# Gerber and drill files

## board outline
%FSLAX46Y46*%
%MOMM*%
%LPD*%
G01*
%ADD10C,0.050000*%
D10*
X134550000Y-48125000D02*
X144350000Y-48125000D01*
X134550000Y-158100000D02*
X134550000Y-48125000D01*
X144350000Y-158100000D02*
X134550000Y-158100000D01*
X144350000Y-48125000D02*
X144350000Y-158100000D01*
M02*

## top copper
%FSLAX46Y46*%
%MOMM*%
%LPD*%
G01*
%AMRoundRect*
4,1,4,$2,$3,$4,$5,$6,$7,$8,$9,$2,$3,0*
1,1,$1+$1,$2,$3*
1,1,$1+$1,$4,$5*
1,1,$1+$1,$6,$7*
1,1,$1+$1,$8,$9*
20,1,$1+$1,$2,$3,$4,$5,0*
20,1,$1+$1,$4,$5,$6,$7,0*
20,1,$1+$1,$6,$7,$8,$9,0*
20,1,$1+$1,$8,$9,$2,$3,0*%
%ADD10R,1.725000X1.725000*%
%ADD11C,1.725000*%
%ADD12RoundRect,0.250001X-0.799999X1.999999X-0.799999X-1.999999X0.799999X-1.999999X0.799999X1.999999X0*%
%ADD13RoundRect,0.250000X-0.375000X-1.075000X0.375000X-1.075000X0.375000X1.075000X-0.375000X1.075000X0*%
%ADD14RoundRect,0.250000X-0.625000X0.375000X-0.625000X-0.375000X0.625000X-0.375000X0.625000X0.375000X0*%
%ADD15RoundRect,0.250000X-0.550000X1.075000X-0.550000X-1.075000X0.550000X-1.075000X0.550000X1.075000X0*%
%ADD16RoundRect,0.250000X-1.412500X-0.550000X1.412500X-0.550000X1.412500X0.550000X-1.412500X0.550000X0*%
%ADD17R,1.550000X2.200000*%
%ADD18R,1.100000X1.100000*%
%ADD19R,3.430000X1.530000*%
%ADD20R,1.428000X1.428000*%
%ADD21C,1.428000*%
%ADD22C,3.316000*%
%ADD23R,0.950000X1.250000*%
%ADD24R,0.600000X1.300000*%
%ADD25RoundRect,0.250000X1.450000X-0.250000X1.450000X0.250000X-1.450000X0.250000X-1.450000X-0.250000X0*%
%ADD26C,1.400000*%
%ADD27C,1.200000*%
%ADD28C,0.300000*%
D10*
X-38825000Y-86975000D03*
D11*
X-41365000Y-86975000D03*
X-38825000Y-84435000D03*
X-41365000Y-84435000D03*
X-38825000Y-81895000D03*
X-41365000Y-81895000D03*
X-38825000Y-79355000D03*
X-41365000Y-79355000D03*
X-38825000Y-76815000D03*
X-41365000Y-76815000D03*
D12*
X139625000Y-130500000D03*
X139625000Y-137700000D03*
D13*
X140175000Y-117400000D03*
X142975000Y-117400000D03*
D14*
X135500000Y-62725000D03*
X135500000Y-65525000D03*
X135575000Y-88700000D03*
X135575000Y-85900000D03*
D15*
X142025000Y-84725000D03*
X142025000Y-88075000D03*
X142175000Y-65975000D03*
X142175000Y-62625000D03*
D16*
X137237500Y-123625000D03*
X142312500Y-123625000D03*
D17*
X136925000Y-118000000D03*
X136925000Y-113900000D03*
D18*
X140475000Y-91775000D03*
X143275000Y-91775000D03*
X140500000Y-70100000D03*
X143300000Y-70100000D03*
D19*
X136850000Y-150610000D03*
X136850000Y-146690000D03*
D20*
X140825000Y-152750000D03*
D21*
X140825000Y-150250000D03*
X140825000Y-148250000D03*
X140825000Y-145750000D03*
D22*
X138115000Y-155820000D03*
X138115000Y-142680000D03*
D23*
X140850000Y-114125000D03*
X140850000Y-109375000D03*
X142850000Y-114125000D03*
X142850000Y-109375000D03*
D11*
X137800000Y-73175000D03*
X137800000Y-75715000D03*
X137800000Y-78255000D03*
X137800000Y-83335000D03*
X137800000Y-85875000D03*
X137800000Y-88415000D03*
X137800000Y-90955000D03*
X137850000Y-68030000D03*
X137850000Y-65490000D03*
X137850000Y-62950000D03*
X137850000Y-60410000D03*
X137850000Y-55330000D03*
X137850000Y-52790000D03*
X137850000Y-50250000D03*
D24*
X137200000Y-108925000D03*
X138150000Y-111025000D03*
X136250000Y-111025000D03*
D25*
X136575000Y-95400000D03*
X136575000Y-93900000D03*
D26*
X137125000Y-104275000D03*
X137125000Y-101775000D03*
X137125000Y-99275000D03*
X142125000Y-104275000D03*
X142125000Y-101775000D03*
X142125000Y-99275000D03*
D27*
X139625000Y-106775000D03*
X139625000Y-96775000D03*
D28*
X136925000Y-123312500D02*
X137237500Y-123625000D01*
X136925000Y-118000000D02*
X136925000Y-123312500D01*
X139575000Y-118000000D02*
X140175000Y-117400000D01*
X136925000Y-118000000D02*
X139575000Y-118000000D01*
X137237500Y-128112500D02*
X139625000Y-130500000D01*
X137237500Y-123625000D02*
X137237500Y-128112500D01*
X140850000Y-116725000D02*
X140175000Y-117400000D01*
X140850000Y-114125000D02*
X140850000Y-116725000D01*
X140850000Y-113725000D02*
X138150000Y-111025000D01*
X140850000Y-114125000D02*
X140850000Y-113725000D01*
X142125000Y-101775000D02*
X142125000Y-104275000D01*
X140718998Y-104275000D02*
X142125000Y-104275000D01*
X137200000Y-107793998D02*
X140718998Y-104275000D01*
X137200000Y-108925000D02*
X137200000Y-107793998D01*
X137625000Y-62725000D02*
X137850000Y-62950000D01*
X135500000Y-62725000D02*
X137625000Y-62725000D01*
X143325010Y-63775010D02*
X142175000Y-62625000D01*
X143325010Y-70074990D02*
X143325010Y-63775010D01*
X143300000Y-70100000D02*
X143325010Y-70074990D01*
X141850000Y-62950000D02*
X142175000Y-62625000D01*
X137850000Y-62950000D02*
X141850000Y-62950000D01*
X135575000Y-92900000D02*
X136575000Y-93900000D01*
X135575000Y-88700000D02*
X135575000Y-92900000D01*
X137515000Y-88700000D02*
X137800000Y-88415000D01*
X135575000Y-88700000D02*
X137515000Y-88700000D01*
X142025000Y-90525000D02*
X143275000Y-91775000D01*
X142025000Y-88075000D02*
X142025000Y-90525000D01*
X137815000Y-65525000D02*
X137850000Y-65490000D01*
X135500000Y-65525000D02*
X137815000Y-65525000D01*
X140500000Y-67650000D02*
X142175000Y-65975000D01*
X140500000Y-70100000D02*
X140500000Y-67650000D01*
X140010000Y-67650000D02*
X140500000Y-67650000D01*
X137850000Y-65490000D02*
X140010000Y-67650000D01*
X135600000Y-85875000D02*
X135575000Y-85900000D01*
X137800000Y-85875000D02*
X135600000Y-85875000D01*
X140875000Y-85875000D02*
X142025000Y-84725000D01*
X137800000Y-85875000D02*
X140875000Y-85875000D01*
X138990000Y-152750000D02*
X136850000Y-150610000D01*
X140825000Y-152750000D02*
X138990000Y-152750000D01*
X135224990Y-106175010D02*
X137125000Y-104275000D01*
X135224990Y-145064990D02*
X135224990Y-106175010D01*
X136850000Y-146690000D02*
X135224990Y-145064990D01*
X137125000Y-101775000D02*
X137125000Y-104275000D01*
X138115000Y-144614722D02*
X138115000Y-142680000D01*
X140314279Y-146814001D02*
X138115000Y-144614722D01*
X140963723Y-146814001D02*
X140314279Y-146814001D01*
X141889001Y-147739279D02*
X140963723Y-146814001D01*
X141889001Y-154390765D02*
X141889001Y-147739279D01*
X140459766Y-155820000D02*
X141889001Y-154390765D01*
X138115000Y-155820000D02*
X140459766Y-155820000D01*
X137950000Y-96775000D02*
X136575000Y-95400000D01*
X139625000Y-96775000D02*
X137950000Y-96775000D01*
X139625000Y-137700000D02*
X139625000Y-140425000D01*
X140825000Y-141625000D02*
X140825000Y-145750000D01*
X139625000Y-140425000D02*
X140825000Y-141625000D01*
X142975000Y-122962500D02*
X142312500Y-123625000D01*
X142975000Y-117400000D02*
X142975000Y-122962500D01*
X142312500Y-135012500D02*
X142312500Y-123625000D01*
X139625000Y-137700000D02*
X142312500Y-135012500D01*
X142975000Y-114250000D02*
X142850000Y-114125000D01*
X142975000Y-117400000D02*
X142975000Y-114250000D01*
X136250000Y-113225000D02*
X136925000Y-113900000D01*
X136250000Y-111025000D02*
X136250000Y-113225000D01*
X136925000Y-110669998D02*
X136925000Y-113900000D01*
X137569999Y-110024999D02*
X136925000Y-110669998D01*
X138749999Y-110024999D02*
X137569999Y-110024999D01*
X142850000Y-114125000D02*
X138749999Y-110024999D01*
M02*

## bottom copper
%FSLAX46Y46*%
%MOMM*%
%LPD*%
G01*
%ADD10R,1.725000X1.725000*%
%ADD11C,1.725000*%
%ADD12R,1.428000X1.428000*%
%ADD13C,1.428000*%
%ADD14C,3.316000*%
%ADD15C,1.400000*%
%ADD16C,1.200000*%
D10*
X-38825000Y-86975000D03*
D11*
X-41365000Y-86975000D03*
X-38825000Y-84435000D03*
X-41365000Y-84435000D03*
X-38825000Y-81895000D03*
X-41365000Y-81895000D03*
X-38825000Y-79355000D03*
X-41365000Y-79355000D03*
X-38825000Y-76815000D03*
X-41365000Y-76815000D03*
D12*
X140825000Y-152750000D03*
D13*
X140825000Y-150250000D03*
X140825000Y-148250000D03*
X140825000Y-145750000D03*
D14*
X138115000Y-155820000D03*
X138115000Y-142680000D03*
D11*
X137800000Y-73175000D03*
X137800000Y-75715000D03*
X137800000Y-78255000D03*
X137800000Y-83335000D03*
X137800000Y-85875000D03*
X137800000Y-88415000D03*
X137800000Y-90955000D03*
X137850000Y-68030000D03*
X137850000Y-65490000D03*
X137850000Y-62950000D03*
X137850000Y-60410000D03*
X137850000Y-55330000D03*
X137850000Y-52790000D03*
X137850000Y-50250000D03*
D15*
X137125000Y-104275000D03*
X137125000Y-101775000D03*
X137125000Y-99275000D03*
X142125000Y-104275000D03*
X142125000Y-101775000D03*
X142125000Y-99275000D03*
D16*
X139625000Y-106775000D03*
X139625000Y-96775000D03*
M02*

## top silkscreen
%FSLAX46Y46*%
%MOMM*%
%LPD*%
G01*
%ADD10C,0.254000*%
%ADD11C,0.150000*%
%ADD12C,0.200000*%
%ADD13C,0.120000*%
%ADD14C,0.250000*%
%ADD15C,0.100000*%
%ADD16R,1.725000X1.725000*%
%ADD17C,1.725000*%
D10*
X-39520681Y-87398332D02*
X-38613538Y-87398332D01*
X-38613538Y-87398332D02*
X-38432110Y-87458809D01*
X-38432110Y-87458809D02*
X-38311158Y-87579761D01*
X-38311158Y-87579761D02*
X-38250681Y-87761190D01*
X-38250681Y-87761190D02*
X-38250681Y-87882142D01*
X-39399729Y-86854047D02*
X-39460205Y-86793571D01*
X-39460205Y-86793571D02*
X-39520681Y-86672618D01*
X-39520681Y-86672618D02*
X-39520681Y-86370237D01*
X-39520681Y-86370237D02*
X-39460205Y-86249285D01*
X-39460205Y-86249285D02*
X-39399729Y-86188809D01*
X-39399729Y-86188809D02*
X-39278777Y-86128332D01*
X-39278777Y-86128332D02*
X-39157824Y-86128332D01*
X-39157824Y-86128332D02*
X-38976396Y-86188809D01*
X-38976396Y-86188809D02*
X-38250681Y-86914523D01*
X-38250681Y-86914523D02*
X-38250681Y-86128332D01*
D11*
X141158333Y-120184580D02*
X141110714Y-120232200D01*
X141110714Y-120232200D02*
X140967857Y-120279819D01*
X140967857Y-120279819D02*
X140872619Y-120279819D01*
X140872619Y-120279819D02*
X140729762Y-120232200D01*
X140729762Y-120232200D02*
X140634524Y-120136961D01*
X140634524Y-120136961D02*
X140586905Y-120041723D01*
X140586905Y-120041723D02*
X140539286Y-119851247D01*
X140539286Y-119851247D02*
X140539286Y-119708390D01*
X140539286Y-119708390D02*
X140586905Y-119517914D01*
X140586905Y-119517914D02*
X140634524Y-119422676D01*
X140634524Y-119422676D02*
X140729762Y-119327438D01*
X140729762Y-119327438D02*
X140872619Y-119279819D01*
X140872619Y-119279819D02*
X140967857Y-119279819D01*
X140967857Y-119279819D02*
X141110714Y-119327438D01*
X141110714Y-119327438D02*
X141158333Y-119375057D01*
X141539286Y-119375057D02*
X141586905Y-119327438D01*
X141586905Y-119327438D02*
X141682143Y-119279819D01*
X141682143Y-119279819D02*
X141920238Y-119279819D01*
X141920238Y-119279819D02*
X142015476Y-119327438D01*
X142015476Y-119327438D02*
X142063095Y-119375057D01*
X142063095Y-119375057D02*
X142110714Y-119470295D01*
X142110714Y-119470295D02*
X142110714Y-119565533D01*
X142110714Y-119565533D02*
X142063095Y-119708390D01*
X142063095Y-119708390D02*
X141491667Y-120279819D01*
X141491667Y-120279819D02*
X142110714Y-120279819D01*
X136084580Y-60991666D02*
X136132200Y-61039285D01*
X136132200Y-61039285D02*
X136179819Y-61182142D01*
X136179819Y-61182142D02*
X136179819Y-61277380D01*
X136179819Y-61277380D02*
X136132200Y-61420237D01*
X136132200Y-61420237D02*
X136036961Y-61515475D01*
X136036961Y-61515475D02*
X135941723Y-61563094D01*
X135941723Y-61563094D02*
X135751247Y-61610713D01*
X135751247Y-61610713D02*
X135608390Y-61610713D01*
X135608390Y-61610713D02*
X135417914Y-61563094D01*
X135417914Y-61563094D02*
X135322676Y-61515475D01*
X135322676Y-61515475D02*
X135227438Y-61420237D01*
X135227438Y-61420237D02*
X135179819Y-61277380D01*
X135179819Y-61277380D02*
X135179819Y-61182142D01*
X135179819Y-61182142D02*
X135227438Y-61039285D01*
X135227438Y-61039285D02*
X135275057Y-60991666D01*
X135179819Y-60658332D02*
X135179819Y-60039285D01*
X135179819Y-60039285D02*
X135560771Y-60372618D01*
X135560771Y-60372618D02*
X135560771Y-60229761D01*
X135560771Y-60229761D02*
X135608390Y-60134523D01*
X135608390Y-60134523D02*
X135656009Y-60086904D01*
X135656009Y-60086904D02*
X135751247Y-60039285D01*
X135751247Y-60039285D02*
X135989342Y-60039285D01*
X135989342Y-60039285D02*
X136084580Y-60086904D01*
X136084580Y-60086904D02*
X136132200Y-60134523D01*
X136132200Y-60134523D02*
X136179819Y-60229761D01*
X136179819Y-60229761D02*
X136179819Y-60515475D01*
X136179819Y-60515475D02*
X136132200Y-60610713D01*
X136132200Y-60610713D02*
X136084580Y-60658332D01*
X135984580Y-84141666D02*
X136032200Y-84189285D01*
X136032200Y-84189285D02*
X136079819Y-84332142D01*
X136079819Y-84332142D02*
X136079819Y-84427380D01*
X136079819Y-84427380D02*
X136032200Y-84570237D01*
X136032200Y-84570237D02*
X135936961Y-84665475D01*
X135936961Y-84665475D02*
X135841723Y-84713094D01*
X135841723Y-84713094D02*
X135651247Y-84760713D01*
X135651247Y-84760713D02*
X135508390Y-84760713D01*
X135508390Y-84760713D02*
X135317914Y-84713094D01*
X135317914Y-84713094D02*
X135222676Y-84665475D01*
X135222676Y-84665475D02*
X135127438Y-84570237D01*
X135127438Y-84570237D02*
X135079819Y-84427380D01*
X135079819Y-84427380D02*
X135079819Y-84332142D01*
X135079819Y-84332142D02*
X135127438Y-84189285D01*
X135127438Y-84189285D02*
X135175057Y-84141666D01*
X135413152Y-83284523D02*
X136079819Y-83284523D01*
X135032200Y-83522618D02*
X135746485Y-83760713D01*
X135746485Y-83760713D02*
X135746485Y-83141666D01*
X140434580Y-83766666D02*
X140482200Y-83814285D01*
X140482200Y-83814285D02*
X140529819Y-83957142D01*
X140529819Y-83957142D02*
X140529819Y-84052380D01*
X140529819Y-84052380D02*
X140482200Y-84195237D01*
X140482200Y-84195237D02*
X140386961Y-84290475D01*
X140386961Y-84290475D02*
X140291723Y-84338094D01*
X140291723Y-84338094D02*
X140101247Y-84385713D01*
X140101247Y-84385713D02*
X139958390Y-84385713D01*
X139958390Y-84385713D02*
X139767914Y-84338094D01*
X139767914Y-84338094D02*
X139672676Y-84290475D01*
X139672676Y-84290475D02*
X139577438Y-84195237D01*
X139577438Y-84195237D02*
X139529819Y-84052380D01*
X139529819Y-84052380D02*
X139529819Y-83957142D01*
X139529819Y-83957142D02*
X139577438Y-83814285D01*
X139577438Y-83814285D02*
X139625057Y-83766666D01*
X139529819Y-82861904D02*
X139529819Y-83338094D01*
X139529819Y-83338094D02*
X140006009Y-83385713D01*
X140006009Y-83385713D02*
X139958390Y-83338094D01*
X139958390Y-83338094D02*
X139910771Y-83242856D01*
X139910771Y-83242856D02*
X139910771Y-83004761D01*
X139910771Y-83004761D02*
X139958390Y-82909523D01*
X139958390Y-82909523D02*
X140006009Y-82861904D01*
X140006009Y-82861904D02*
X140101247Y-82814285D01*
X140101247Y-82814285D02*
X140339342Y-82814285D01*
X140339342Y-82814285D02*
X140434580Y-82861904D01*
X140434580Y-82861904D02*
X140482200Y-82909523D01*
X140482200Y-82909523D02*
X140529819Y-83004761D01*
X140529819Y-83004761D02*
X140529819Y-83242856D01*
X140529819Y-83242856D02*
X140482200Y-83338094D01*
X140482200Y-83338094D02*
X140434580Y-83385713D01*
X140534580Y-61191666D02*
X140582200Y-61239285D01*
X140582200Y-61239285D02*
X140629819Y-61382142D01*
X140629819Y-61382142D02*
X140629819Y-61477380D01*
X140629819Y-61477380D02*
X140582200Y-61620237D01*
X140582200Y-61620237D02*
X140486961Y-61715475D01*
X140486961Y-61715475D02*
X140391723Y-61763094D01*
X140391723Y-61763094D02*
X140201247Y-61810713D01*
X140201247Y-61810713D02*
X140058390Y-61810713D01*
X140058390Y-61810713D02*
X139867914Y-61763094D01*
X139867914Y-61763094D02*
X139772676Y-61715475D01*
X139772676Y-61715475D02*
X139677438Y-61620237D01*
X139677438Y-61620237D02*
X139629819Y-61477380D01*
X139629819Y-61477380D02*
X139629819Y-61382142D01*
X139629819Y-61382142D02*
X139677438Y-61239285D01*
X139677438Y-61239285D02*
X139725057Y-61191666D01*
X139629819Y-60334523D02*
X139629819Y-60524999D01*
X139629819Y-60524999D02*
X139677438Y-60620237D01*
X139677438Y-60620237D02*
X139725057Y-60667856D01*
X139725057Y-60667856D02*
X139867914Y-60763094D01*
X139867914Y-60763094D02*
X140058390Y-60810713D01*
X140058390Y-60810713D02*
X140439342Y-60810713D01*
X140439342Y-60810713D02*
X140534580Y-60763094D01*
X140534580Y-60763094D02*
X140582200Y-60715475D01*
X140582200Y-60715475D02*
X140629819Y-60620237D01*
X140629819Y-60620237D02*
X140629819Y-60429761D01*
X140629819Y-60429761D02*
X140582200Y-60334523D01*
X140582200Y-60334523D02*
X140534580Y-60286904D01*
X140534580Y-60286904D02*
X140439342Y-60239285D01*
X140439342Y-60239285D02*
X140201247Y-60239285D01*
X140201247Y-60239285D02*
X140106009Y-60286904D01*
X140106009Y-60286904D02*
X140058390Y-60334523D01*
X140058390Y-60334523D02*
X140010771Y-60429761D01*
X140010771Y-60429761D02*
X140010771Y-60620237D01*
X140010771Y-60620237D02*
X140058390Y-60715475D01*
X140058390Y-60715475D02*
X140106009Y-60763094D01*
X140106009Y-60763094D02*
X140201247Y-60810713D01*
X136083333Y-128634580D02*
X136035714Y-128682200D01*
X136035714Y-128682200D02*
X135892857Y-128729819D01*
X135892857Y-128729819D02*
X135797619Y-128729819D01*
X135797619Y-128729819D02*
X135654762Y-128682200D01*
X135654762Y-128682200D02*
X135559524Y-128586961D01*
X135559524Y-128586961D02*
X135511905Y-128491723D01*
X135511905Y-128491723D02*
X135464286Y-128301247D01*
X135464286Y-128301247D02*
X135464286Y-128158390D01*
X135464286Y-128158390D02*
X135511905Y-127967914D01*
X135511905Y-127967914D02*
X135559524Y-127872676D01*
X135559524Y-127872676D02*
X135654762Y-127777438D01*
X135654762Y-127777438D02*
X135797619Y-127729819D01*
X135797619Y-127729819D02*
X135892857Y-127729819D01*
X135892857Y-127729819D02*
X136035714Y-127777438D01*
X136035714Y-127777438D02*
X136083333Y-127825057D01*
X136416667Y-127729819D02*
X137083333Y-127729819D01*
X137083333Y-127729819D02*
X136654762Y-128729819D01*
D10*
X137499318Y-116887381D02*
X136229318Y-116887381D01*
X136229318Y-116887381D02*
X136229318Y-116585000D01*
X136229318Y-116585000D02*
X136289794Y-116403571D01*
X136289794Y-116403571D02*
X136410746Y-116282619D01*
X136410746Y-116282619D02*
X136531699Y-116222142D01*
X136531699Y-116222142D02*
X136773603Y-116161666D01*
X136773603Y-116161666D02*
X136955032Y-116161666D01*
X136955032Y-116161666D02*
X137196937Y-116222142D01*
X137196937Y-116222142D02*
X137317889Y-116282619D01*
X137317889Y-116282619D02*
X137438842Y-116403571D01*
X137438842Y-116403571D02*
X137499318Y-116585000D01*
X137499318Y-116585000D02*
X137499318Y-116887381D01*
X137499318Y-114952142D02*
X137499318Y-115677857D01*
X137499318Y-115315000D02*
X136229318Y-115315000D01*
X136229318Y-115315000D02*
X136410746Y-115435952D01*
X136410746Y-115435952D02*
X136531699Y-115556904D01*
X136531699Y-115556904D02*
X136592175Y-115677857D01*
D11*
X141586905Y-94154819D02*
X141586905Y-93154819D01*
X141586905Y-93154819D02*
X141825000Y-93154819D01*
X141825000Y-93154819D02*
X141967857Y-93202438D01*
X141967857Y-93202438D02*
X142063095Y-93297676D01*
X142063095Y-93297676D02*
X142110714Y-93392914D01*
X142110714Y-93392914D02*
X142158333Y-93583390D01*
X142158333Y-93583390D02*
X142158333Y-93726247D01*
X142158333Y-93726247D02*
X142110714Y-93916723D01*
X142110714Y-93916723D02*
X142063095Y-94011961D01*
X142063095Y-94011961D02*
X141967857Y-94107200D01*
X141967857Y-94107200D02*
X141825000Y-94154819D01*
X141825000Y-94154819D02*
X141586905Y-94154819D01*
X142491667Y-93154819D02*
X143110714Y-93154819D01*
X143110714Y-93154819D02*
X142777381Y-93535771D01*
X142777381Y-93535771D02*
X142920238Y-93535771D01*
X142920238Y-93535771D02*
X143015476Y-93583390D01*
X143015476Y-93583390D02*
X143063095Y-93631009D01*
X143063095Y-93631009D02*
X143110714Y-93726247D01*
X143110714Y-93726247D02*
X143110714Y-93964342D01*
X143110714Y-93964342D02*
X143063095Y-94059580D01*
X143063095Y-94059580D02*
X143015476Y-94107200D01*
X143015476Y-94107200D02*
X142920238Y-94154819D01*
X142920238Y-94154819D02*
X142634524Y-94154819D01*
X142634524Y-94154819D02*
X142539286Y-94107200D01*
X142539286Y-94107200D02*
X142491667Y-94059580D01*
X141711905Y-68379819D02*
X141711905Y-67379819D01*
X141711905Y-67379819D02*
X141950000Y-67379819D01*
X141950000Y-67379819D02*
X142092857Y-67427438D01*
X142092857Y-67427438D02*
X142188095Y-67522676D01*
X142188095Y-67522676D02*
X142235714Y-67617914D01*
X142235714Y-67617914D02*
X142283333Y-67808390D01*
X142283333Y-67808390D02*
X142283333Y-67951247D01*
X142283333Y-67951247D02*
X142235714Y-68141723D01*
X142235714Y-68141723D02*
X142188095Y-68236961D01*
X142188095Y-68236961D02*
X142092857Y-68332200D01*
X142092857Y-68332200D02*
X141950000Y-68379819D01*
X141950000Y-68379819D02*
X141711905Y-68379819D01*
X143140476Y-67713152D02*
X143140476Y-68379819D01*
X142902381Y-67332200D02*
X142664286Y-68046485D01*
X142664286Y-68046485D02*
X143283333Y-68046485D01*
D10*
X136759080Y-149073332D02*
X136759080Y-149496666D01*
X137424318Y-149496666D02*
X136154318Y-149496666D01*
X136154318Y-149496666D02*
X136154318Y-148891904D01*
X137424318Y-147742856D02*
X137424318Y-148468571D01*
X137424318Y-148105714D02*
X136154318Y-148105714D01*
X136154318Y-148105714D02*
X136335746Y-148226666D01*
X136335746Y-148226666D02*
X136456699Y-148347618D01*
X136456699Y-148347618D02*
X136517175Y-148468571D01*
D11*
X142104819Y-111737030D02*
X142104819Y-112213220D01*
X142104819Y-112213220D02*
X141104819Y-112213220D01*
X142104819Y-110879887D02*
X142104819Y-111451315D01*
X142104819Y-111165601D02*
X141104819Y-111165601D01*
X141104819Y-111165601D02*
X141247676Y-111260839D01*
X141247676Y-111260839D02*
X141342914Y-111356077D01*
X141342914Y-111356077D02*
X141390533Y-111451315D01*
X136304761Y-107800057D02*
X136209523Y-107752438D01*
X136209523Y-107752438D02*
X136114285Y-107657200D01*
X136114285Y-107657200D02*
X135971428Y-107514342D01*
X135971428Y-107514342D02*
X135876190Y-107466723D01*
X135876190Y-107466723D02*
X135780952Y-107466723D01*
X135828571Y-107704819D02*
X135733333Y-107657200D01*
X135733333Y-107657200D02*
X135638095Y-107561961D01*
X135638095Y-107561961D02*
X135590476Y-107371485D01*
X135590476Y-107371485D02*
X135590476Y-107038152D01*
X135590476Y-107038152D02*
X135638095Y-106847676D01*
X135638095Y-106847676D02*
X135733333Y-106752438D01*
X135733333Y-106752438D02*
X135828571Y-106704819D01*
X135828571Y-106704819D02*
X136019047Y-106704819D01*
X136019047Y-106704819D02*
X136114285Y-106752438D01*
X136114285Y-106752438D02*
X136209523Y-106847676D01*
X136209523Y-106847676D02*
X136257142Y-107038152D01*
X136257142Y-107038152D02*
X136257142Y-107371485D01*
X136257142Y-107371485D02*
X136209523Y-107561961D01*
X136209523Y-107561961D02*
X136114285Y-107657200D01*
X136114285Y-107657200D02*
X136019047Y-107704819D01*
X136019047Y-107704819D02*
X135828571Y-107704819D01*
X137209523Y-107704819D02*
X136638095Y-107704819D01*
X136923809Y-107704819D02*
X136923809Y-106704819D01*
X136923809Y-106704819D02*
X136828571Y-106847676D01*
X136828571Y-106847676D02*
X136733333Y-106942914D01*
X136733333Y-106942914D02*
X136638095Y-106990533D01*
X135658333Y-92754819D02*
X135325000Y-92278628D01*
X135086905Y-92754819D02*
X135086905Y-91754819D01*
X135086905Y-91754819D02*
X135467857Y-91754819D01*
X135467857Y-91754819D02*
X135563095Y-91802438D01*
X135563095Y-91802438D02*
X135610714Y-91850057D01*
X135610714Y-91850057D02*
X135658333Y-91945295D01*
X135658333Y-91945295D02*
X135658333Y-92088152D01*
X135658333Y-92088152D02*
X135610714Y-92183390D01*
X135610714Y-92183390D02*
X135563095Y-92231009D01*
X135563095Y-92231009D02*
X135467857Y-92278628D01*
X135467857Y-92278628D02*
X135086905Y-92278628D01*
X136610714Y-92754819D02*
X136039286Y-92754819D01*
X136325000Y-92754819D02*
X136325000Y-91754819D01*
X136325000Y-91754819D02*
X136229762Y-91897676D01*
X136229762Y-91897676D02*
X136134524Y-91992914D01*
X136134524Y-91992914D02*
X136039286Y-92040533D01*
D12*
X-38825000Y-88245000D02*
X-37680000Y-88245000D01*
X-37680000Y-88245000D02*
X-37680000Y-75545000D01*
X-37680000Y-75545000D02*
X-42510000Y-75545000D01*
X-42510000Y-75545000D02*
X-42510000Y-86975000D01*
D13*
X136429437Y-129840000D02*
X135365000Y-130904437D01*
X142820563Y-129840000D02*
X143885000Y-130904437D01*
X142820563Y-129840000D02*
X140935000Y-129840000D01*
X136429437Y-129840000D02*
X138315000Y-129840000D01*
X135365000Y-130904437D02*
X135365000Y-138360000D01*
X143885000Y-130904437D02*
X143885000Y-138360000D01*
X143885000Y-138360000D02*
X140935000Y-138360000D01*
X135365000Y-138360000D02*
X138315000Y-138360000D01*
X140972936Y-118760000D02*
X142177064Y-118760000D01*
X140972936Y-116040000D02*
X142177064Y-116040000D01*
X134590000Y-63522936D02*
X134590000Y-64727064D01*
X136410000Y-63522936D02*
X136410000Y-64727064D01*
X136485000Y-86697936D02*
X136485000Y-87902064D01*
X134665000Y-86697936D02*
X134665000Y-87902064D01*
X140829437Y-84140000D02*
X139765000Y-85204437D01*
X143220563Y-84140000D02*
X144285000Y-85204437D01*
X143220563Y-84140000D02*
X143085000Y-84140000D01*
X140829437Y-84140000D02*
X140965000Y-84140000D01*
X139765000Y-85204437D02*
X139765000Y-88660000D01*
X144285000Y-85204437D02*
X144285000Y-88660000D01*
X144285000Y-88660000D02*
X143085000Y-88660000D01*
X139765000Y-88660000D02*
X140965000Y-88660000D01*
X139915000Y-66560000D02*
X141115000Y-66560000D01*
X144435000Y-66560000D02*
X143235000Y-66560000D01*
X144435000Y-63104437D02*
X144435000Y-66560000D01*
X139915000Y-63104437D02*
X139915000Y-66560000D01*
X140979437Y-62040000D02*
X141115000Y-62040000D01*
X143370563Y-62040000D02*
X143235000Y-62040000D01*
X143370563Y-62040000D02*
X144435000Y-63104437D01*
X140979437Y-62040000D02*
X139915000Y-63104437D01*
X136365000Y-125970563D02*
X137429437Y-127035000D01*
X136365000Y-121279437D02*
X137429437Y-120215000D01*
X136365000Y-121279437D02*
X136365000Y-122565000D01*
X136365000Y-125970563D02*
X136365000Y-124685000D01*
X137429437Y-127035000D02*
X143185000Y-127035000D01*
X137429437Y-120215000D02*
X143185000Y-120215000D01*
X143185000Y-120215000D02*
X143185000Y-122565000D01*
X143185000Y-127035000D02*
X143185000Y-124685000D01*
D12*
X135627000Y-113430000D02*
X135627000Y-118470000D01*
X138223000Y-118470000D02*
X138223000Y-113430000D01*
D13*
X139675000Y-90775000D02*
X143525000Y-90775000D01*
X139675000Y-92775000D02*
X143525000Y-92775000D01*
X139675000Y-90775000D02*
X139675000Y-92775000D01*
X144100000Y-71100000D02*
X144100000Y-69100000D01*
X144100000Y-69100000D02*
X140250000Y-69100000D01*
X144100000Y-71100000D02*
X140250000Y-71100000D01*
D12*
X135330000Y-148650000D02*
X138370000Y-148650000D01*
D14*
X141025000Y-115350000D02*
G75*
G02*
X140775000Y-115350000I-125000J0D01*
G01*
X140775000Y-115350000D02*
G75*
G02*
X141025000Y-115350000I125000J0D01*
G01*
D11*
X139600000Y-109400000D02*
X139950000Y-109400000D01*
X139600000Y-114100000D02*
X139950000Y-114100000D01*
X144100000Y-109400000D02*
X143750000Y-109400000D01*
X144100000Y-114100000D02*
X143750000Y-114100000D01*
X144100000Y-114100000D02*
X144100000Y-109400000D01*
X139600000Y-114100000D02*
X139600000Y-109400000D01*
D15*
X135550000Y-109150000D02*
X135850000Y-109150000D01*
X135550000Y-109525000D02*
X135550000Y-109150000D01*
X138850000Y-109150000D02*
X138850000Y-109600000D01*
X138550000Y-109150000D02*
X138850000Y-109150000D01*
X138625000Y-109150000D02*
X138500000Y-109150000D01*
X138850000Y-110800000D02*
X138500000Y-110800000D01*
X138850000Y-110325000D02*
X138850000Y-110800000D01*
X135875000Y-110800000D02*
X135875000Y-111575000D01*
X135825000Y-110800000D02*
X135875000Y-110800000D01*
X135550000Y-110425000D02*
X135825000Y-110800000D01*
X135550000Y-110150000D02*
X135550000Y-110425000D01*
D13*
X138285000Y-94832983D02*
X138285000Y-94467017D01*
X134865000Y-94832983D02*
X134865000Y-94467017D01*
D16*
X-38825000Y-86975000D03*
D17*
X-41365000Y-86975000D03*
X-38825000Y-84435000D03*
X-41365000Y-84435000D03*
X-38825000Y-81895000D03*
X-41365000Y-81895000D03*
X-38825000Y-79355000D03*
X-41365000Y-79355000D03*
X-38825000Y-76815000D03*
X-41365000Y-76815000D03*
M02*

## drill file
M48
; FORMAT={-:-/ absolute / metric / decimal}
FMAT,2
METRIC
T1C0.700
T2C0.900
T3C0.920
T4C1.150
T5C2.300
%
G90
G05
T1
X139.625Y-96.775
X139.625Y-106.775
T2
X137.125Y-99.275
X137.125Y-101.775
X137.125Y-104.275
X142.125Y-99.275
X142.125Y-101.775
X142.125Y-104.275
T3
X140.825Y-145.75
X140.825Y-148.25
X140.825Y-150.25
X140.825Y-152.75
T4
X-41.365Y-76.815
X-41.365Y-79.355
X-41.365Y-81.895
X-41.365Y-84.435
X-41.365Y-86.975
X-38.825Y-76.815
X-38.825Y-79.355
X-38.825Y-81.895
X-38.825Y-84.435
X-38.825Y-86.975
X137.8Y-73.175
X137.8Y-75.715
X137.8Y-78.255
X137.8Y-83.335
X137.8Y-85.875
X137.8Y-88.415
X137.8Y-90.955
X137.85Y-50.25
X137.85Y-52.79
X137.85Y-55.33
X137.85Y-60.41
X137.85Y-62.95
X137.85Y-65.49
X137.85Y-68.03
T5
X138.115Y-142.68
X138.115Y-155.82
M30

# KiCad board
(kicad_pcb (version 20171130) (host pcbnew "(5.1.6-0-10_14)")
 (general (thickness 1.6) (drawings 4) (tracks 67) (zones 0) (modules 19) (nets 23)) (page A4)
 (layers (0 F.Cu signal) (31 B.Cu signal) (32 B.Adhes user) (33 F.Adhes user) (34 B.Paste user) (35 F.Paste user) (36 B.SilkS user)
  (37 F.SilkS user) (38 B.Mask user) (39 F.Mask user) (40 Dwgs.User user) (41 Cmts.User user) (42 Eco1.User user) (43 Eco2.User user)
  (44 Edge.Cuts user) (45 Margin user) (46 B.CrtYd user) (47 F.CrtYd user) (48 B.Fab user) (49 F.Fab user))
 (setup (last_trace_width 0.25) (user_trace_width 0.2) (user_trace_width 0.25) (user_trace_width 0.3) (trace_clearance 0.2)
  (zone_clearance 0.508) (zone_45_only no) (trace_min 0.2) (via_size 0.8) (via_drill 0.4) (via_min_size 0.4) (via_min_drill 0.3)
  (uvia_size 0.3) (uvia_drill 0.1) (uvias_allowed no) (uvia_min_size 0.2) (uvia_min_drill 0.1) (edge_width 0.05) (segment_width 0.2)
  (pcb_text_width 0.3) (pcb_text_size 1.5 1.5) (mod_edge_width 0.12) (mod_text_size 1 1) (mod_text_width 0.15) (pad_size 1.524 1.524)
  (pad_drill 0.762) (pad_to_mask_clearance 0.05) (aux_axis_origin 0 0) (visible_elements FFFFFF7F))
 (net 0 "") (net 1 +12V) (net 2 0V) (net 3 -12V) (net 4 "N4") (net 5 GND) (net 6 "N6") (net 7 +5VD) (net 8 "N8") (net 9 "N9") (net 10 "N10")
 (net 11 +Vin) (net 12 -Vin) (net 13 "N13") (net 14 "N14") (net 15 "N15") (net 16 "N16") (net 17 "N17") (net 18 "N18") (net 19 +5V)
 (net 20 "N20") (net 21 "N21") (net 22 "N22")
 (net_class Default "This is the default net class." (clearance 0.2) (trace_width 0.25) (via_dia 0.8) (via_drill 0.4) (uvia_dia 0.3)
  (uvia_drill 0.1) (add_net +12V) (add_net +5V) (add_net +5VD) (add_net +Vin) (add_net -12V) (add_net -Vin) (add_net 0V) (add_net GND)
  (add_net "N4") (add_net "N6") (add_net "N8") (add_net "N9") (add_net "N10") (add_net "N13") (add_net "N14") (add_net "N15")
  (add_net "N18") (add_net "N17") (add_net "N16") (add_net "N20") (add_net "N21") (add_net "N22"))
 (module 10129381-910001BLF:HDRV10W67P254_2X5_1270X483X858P (layer F.Cu) (at -38.825 86.975 90)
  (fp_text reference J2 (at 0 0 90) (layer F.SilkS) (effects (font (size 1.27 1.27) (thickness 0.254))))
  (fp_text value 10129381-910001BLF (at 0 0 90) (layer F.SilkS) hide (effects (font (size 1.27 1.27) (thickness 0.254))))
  (fp_line (start -1.27 0) (end -1.27 1.145) (layer F.SilkS) (width 0.2))
  (fp_line (start -1.27 1.145) (end 11.43 1.145) (layer F.SilkS) (width 0.2))
  (fp_line (start 11.43 1.145) (end 11.43 -3.685) (layer F.SilkS) (width 0.2))
  (fp_line (start 11.43 -3.685) (end 0 -3.685) (layer F.SilkS) (width 0.2))
  (pad 1 thru_hole rect (at 0 0 180) (size 1.725 1.725) (drill 1.15) (layers *.Cu *.Mask F.SilkS) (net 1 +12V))
  (pad 2 thru_hole circle (at 0 -2.54 180) (size 1.725 1.725) (drill 1.15) (layers *.Cu *.Mask F.SilkS) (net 1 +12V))
  (pad 3 thru_hole circle (at 2.54 0 180) (size 1.725 1.725) (drill 1.15) (layers *.Cu *.Mask F.SilkS) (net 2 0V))
  (pad 4 thru_hole circle (at 2.54 -2.54 180) (size 1.725 1.725) (drill 1.15) (layers *.Cu *.Mask F.SilkS) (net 2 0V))
  (pad 5 thru_hole circle (at 5.08 0 180) (size 1.725 1.725) (drill 1.15) (layers *.Cu *.Mask F.SilkS) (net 2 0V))
  (pad 6 thru_hole circle (at 5.08 -2.54 180) (size 1.725 1.725) (drill 1.15) (layers *.Cu *.Mask F.SilkS) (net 2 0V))
  (pad 7 thru_hole circle (at 7.62 0 180) (size 1.725 1.725) (drill 1.15) (layers *.Cu *.Mask F.SilkS) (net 2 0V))
  (pad 8 thru_hole circle (at 7.62 -2.54 180) (size 1.725 1.725) (drill 1.15) (layers *.Cu *.Mask F.SilkS) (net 2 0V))
  (pad 9 thru_hole circle (at 10.16 0 180) (size 1.725 1.725) (drill 1.15) (layers *.Cu *.Mask F.SilkS) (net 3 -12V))
  (pad 10 thru_hole circle (at 10.16 -2.54 180) (size 1.725 1.725) (drill 1.15) (layers *.Cu *.Mask F.SilkS) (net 3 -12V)))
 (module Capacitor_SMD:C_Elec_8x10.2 (layer F.Cu) (at 139.625 134.1 270)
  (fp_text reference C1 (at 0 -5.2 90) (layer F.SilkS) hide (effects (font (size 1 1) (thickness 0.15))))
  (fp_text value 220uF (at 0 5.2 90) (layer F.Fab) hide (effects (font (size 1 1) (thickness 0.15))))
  (fp_line (start -4.26 3.195563) (end -3.195563 4.26) (layer F.SilkS) (width 0.12))
  (fp_line (start -4.26 -3.195563) (end -3.195563 -4.26) (layer F.SilkS) (width 0.12))
  (fp_line (start -4.26 -3.195563) (end -4.26 -1.31) (layer F.SilkS) (width 0.12))
  (fp_line (start -4.26 3.195563) (end -4.26 1.31) (layer F.SilkS) (width 0.12))
  (fp_line (start -3.195563 4.26) (end 4.26 4.26) (layer F.SilkS) (width 0.12))
  (fp_line (start -3.195563 -4.26) (end 4.26 -4.26) (layer F.SilkS) (width 0.12))
  (fp_line (start 4.26 -4.26) (end 4.26 -1.31) (layer F.SilkS) (width 0.12))
  (fp_line (start 4.26 4.26) (end 4.26 1.31) (layer F.SilkS) (width 0.12))
  (pad 1 smd roundrect (at -3.6 0 270) (size 4.5 2.1) (layers F.Cu F.Paste F.Mask) (roundrect_rratio 0.119048) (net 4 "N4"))
  (pad 2 smd roundrect (at 3.6 0 270) (size 4.5 2.1) (layers F.Cu F.Paste F.Mask) (roundrect_rratio 0.119048) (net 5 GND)))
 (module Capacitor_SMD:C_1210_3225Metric (layer F.Cu) (at 141.575 117.4)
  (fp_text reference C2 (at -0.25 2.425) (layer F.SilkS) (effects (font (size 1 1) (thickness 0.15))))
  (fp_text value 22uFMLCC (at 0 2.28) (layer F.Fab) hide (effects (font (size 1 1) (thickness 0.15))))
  (fp_line (start -0.602064 1.36) (end 0.602064 1.36) (layer F.SilkS) (width 0.12))
  (fp_line (start -0.602064 -1.36) (end 0.602064 -1.36) (layer F.SilkS) (width 0.12))
  (pad 1 smd roundrect (at -1.4 0) (size 1.25 2.65) (layers F.Cu F.Paste F.Mask) (roundrect_rratio 0.2) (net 4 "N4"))
  (pad 2 smd roundrect (at 1.4 0) (size 1.25 2.65) (layers F.Cu F.Paste F.Mask) (roundrect_rratio 0.2) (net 5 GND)))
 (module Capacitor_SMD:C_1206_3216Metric (layer F.Cu) (at 135.5 64.125 270)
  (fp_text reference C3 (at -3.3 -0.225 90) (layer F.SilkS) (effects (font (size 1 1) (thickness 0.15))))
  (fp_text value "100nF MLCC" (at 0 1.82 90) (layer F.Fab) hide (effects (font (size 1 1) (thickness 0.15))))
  (fp_line (start -0.602064 0.91) (end 0.602064 0.91) (layer F.SilkS) (width 0.12))
  (fp_line (start -0.602064 -0.91) (end 0.602064 -0.91) (layer F.SilkS) (width 0.12))
  (pad 1 smd roundrect (at -1.4 0 270) (size 1.25 1.75) (layers F.Cu F.Paste F.Mask) (roundrect_rratio 0.2) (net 2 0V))
  (pad 2 smd roundrect (at 1.4 0 270) (size 1.25 1.75) (layers F.Cu F.Paste F.Mask) (roundrect_rratio 0.2) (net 3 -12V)))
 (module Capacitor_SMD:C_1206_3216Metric (layer F.Cu) (at 135.575 87.3 270)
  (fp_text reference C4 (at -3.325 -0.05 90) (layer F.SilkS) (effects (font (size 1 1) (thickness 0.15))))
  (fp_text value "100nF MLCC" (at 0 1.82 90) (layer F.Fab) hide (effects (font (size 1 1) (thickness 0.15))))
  (fp_line (start -0.602064 -0.91) (end 0.602064 -0.91) (layer F.SilkS) (width 0.12))
  (fp_line (start -0.602064 0.91) (end 0.602064 0.91) (layer F.SilkS) (width 0.12))
  (pad 2 smd roundrect (at 1.4 0 270) (size 1.25 1.75) (layers F.Cu F.Paste F.Mask) (roundrect_rratio 0.2) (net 2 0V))
  (pad 1 smd roundrect (at -1.4 0 270) (size 1.25 1.75) (layers F.Cu F.Paste F.Mask) (roundrect_rratio 0.2) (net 1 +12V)))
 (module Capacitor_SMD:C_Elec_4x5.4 (layer F.Cu) (at 142.025 86.4 270)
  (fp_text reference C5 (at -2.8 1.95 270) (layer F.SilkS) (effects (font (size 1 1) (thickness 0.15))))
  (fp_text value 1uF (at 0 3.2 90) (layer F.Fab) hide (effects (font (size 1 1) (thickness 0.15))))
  (fp_line (start -2.26 1.195563) (end -1.195563 2.26) (layer F.SilkS) (width 0.12))
  (fp_line (start -2.26 -1.195563) (end -1.195563 -2.26) (layer F.SilkS) (width 0.12))
  (fp_line (start -2.26 -1.195563) (end -2.26 -1.06) (layer F.SilkS) (width 0.12))
  (fp_line (start -2.26 1.195563) (end -2.26 1.06) (layer F.SilkS) (width 0.12))
  (fp_line (start -1.195563 2.26) (end 2.26 2.26) (layer F.SilkS) (width 0.12))
  (fp_line (start -1.195563 -2.26) (end 2.26 -2.26) (layer F.SilkS) (width 0.12))
  (fp_line (start 2.26 -2.26) (end 2.26 -1.06) (layer F.SilkS) (width 0.12))
  (fp_line (start 2.26 2.26) (end 2.26 1.06) (layer F.SilkS) (width 0.12))
  (pad 1 smd roundrect (at -1.675 0 270) (size 2.65 1.6) (layers F.Cu F.Paste F.Mask) (roundrect_rratio 0.15625) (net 1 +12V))
  (pad 2 smd roundrect (at 1.675 0 270) (size 2.65 1.6) (layers F.Cu F.Paste F.Mask) (roundrect_rratio 0.15625) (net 2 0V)))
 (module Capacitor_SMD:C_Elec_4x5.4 (layer F.Cu) (at 142.175 64.3 270)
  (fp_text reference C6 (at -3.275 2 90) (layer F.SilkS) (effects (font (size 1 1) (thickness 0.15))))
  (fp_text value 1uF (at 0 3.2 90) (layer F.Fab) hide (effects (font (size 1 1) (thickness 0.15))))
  (fp_line (start 2.26 2.26) (end 2.26 1.06) (layer F.SilkS) (width 0.12))
  (fp_line (start 2.26 -2.26) (end 2.26 -1.06) (layer F.SilkS) (width 0.12))
  (fp_line (start -1.195563 -2.26) (end 2.26 -2.26) (layer F.SilkS) (width 0.12))
  (fp_line (start -1.195563 2.26) (end 2.26 2.26) (layer F.SilkS) (width 0.12))
  (fp_line (start -2.26 1.195563) (end -2.26 1.06) (layer F.SilkS) (width 0.12))
  (fp_line (start -2.26 -1.195563) (end -2.26 -1.06) (layer F.SilkS) (width 0.12))
  (fp_line (start -2.26 -1.195563) (end -1.195563 -2.26) (layer F.SilkS) (width 0.12))
  (fp_line (start -2.26 1.195563) (end -1.195563 2.26) (layer F.SilkS) (width 0.12))
  (pad 2 smd roundrect (at 1.675 0 270) (size 2.65 1.6) (layers F.Cu F.Paste F.Mask) (roundrect_rratio 0.15625) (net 3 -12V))
  (pad 1 smd roundrect (at -1.675 0 270) (size 2.65 1.6) (layers F.Cu F.Paste F.Mask) (roundrect_rratio 0.15625) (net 2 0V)))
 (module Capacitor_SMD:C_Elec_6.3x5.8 (layer F.Cu) (at 139.775 123.625)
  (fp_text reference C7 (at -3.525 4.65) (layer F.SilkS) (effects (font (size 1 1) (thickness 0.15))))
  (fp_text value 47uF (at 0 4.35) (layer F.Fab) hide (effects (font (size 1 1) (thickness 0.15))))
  (fp_line (start -3.41 2.345563) (end -2.345563 3.41) (layer F.SilkS) (width 0.12))
  (fp_line (start -3.41 -2.345563) (end -2.345563 -3.41) (layer F.SilkS) (width 0.12))
  (fp_line (start -3.41 -2.345563) (end -3.41 -1.06) (layer F.SilkS) (width 0.12))
  (fp_line (start -3.41 2.345563) (end -3.41 1.06) (layer F.SilkS) (width 0.12))
  (fp_line (start -2.345563 3.41) (end 3.41 3.41) (layer F.SilkS) (width 0.12))
  (fp_line (start -2.345563 -3.41) (end 3.41 -3.41) (layer F.SilkS) (width 0.12))
  (fp_line (start 3.41 -3.41) (end 3.41 -1.06) (layer F.SilkS) (width 0.12))
  (fp_line (start 3.41 3.41) (end 3.41 1.06) (layer F.SilkS) (width 0.12))
  (pad 1 smd roundrect (at -2.5375 0) (size 3.325 1.6) (layers F.Cu F.Paste F.Mask) (roundrect_rratio 0.15625) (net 4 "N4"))
  (pad 2 smd roundrect (at 2.5375 0) (size 3.325 1.6) (layers F.Cu F.Paste F.Mask) (roundrect_rratio 0.15625) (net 5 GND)))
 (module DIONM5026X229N (layer F.Cu) (at 136.925 115.95 90)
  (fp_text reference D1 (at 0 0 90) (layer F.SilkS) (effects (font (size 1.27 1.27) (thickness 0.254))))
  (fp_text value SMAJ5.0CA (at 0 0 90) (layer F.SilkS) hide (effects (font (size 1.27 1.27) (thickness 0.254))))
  (fp_line (start 2.52 -1.298) (end -2.52 -1.298) (layer F.SilkS) (width 0.2))
  (fp_line (start -2.52 1.298) (end 2.52 1.298) (layer F.SilkS) (width 0.2))
  (pad 1 smd rect (at -2.05 0 180) (size 1.55 2.2) (layers F.Cu F.Paste F.Mask) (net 4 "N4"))
  (pad 2 smd rect (at 2.05 0 180) (size 1.55 2.2) (layers F.Cu F.Paste F.Mask) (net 5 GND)))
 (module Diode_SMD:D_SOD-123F (layer F.Cu) (at 141.875 91.775)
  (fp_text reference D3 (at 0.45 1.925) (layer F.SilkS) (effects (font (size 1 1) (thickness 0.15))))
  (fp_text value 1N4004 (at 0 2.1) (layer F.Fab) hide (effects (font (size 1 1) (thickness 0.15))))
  (fp_line (start -2.2 -1) (end 1.65 -1) (layer F.SilkS) (width 0.12))
  (fp_line (start -2.2 1) (end 1.65 1) (layer F.SilkS) (width 0.12))
  (fp_line (start -2.2 -1) (end -2.2 1) (layer F.SilkS) (width 0.12))
  (pad 1 smd rect (at -1.4 0) (size 1.1 1.1) (layers F.Cu F.Paste F.Mask) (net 1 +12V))
  (pad 2 smd rect (at 1.4 0) (size 1.1 1.1) (layers F.Cu F.Paste F.Mask) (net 2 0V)))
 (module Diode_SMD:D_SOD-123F (layer F.Cu) (at 141.9 70.1 180)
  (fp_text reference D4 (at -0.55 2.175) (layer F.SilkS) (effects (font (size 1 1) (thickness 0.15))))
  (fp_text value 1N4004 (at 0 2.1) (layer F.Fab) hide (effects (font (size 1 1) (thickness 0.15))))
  (fp_line (start -2.2 -1) (end -2.2 1) (layer F.SilkS) (width 0.12))
  (fp_line (start -2.2 1) (end 1.65 1) (layer F.SilkS) (width 0.12))
  (fp_line (start -2.2 -1) (end 1.65 -1) (layer F.SilkS) (width 0.12))
  (pad 2 smd rect (at 1.4 0 180) (size 1.1 1.1) (layers F.Cu F.Paste F.Mask) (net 3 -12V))
  (pad 1 smd rect (at -1.4 0 180) (size 1.1 1.1) (layers F.Cu F.Paste F.Mask) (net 2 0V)))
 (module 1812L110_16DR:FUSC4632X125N (layer F.Cu) (at 136.85 148.65 90)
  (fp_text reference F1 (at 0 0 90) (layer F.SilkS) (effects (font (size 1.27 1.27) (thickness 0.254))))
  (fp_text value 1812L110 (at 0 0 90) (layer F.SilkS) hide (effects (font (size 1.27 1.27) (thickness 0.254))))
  (fp_line (start 0 -1.52) (end 0 1.52) (layer F.SilkS) (width 0.2))
  (pad 1 smd rect (at -1.96 0 90) (size 1.53 3.43) (layers F.Cu F.Paste F.Mask) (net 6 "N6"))
  (pad 2 smd rect (at 1.96 0 90) (size 1.53 3.43) (layers F.Cu F.Paste F.Mask) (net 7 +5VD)))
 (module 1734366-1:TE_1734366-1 (layer B.Cu) (at 140.825 152.75 90)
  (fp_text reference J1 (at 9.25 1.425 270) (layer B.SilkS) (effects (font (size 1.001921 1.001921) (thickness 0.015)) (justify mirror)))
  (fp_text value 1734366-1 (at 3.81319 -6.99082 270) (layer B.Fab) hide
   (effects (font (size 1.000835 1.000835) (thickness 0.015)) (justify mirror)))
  (pad 1 thru_hole rect (at 0 0 90) (size 1.428 1.428) (drill 0.92) (layers *.Cu *.Mask) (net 6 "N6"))
  (pad 2 thru_hole circle (at 2.5 0 90) (size 1.428 1.428) (drill 0.92) (layers *.Cu *.Mask) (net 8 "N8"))
  (pad 3 thru_hole circle (at 4.5 0 90) (size 1.428 1.428) (drill 0.92) (layers *.Cu *.Mask) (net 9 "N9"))
  (pad 4 thru_hole circle (at 7 0 90) (size 1.428 1.428) (drill 0.92) (layers *.Cu *.Mask) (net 5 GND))
  (pad SH1 thru_hole circle (at -3.07 -2.71 90) (size 3.316 3.316) (drill 2.3) (layers *.Cu *.Mask) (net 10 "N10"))
  (pad SH2 thru_hole circle (at 10.07 -2.71 90) (size 3.316 3.316) (drill 2.3) (layers *.Cu *.Mask) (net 10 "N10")))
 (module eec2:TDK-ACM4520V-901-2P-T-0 (layer F.Cu) (at 141.85 111.75 90)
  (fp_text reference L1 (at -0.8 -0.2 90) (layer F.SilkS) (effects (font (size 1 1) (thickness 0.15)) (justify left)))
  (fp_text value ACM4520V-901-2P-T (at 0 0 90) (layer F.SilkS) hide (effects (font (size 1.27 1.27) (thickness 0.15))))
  (fp_circle (center -3.6 -0.95) (end -3.475 -0.95) (layer F.SilkS) (width 0.25))
  (fp_line (start 2.35 -2.25) (end 2.35 -1.9) (layer F.SilkS) (width 0.15))
  (fp_line (start -2.35 -2.25) (end -2.35 -1.9) (layer F.SilkS) (width 0.15))
  (fp_line (start 2.35 2.25) (end 2.35 1.9) (layer F.SilkS) (width 0.15))
  (fp_line (start -2.35 2.25) (end -2.35 1.9) (layer F.SilkS) (width 0.15))
  (fp_line (start -2.35 2.25) (end 2.35 2.25) (layer F.SilkS) (width 0.15))
  (fp_line (start -2.35 -2.25) (end 2.35 -2.25) (layer F.SilkS) (width 0.15))
  (pad 1 smd rect (at -2.375 -1 90) (size 1.25 0.95) (layers F.Cu F.Paste F.Mask) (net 4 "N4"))
  (pad 4 smd rect (at 2.375 -1 90) (size 1.25 0.95) (layers F.Cu F.Paste F.Mask) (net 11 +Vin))
  (pad 2 smd rect (at -2.375 1 90) (size 1.25 0.95) (layers F.Cu F.Paste F.Mask) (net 5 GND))
  (pad 3 smd rect (at 2.375 1 90) (size 1.25 0.95) (layers F.Cu F.Paste F.Mask) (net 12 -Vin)))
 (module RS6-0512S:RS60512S (layer B.Cu) (at 137.8 73.175 270)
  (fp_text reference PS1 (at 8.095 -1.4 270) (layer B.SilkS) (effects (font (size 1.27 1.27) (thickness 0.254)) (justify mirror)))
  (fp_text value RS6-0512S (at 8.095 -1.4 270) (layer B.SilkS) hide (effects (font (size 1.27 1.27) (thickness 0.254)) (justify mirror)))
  (pad 1 thru_hole circle (at 0 0 180) (size 1.725 1.725) (drill 1.15) (layers *.Cu *.Mask B.SilkS) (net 12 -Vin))
  (pad 2 thru_hole circle (at 2.54 0 180) (size 1.725 1.725) (drill 1.15) (layers *.Cu *.Mask B.SilkS) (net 11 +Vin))
  (pad 3 thru_hole circle (at 5.08 0 180) (size 1.725 1.725) (drill 1.15) (layers *.Cu *.Mask B.SilkS) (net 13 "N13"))
  (pad 5 thru_hole circle (at 10.16 0 180) (size 1.725 1.725) (drill 1.15) (layers *.Cu *.Mask B.SilkS) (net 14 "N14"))
  (pad 6 thru_hole circle (at 12.7 0 180) (size 1.725 1.725) (drill 1.15) (layers *.Cu *.Mask B.SilkS) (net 1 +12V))
  (pad 7 thru_hole circle (at 15.24 0 180) (size 1.725 1.725) (drill 1.15) (layers *.Cu *.Mask B.SilkS) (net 2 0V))
  (pad 8 thru_hole circle (at 17.78 0 180) (size 1.725 1.725) (drill 1.15) (layers *.Cu *.Mask B.SilkS) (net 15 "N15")))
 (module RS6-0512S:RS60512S (layer B.Cu) (at 137.85 50.25 270)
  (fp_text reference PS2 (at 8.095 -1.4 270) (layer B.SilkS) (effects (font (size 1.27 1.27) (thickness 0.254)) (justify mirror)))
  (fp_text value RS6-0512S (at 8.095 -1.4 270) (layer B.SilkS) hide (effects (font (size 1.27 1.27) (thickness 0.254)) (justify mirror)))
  (pad 8 thru_hole circle (at 17.78 0 180) (size 1.725 1.725) (drill 1.15) (layers *.Cu *.Mask B.SilkS) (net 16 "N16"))
  (pad 7 thru_hole circle (at 15.24 0 180) (size 1.725 1.725) (drill 1.15) (layers *.Cu *.Mask B.SilkS) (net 3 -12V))
  (pad 6 thru_hole circle (at 12.7 0 180) (size 1.725 1.725) (drill 1.15) (layers *.Cu *.Mask B.SilkS) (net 2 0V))
  (pad 5 thru_hole circle (at 10.16 0 180) (size 1.725 1.725) (drill 1.15) (layers *.Cu *.Mask B.SilkS) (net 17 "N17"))
  (pad 3 thru_hole circle (at 5.08 0 180) (size 1.725 1.725) (drill 1.15) (layers *.Cu *.Mask B.SilkS) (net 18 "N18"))
  (pad 2 thru_hole circle (at 2.54 0 180) (size 1.725 1.725) (drill 1.15) (layers *.Cu *.Mask B.SilkS) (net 11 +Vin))
  (pad 1 thru_hole circle (at 0 0 180) (size 1.725 1.725) (drill 1.15) (layers *.Cu *.Mask B.SilkS) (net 12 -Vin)))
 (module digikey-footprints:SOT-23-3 (layer F.Cu) (at 137.2 109.975 90)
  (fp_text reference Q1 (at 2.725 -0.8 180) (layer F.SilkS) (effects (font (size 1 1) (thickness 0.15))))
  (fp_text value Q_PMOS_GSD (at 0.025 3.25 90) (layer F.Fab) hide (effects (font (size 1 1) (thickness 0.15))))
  (fp_line (start 0.825 -1.65) (end 0.825 -1.35) (layer F.SilkS) (width 0.1))
  (fp_line (start 0.45 -1.65) (end 0.825 -1.65) (layer F.SilkS) (width 0.1))
  (fp_line (start 0.825 1.65) (end 0.375 1.65) (layer F.SilkS) (width 0.1))
  (fp_line (start 0.825 1.35) (end 0.825 1.65) (layer F.SilkS) (width 0.1))
  (fp_line (start 0.825 1.425) (end 0.825 1.3) (layer F.SilkS) (width 0.1))
  (fp_line (start -0.825 1.65) (end -0.825 1.3) (layer F.SilkS) (width 0.1))
  (fp_line (start -0.35 1.65) (end -0.825 1.65) (layer F.SilkS) (width 0.1))
  (fp_line (start -0.825 -1.325) (end -1.6 -1.325) (layer F.SilkS) (width 0.1))
  (fp_line (start -0.825 -1.375) (end -0.825 -1.325) (layer F.SilkS) (width 0.1))
  (fp_line (start -0.45 -1.65) (end -0.825 -1.375) (layer F.SilkS) (width 0.1))
  (fp_line (start -0.175 -1.65) (end -0.45 -1.65) (layer F.SilkS) (width 0.1))
  (pad 3 smd rect (at 1.05 0 90) (size 1.3 0.6) (layers F.Cu F.Paste F.Mask) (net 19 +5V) (solder_mask_margin 0.07))
  (pad 2 smd rect (at -1.05 0.95 90) (size 1.3 0.6) (layers F.Cu F.Paste F.Mask) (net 4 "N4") (solder_mask_margin 0.07))
  (pad 1 smd rect (at -1.05 -0.95 90) (size 1.3 0.6) (layers F.Cu F.Paste F.Mask) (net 5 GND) (solder_mask_margin 0.07)))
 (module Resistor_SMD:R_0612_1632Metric (layer F.Cu) (at 136.575 94.65 90)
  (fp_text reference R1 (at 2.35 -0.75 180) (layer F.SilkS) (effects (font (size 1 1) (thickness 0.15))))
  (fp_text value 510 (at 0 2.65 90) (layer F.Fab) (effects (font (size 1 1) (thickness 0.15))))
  (fp_line (start -0.182983 1.71) (end 0.182983 1.71) (layer F.SilkS) (width 0.12))
  (fp_line (start -0.182983 -1.71) (end 0.182983 -1.71) (layer F.SilkS) (width 0.12))
  (pad 1 smd roundrect (at -0.75 0 90) (size 1 3.4) (layers F.Cu F.Paste F.Mask) (roundrect_rratio 0.25) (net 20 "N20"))
  (pad 2 smd roundrect (at 0.75 0 90) (size 1 3.4) (layers F.Cu F.Paste F.Mask) (roundrect_rratio 0.25) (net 2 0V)))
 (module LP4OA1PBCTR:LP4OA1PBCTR (layer B.Cu) (at 137.125 104.275 270)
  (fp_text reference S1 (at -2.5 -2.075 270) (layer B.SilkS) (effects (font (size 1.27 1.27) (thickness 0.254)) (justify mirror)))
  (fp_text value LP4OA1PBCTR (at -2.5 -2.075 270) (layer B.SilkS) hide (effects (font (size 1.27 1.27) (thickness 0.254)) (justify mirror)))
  (pad 1 thru_hole circle (at 0 0 180) (size 1.4 1.4) (drill 0.9) (layers *.Cu *.Mask B.SilkS) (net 7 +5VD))
  (pad 2 thru_hole circle (at -2.5 0 180) (size 1.4 1.4) (drill 0.9) (layers *.Cu *.Mask B.SilkS) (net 7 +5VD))
  (pad 3 thru_hole circle (at -5 0 180) (size 1.4 1.4) (drill 0.9) (layers *.Cu *.Mask B.SilkS) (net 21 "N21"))
  (pad 4 thru_hole circle (at 0 -5 180) (size 1.4 1.4) (drill 0.9) (layers *.Cu *.Mask B.SilkS) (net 19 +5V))
  (pad 5 thru_hole circle (at -2.5 -5 180) (size 1.4 1.4) (drill 0.9) (layers *.Cu *.Mask B.SilkS) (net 19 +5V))
  (pad 6 thru_hole circle (at -5 -5 180) (size 1.4 1.4) (drill 0.9) (layers *.Cu *.Mask B.SilkS) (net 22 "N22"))
  (pad L1 thru_hole circle (at 2.5 -2.5 180) (size 1.2 1.2) (drill 0.7) (layers *.Cu *.Mask B.SilkS) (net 1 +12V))
  (pad L2 thru_hole circle (at -7.5 -2.5 180) (size 1.2 1.2) (drill 0.7) (layers *.Cu *.Mask B.SilkS) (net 20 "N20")))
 (gr_line (start 134.55 48.125) (end 144.35 48.125) (layer Edge.Cuts) (width 0.05))
 (gr_line (start 134.55 158.1) (end 134.55 48.125) (layer Edge.Cuts) (width 0.05))
 (gr_line (start 144.35 158.1) (end 134.55 158.1) (layer Edge.Cuts) (width 0.05))
 (gr_line (start 144.35 48.125) (end 144.35 158.1) (layer Edge.Cuts) (width 0.05))
 (segment (start 136.925 123.3125) (end 137.2375 123.625) (width 0.3) (layer F.Cu) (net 4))
 (segment (start 136.925 118) (end 136.925 123.3125) (width 0.3) (layer F.Cu) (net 4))
 (segment (start 139.575 118) (end 140.175 117.4) (width 0.3) (layer F.Cu) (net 4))
 (segment (start 136.925 118) (end 139.575 118) (width 0.3) (layer F.Cu) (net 4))
 (segment (start 137.2375 128.1125) (end 139.625 130.5) (width 0.3) (layer F.Cu) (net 4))
 (segment (start 137.2375 123.625) (end 137.2375 128.1125) (width 0.3) (layer F.Cu) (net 4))
 (segment (start 140.85 116.725) (end 140.175 117.4) (width 0.3) (layer F.Cu) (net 4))
 (segment (start 140.85 114.125) (end 140.85 116.725) (width 0.3) (layer F.Cu) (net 4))
 (segment (start 140.85 113.725) (end 138.15 111.025) (width 0.3) (layer F.Cu) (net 4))
 (segment (start 140.85 114.125) (end 140.85 113.725) (width 0.3) (layer F.Cu) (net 4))
 (segment (start 142.125 101.775) (end 142.125 104.275) (width 0.3) (layer F.Cu) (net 19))
 (segment (start 140.718998 104.275) (end 142.125 104.275) (width 0.3) (layer F.Cu) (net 19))
 (segment (start 137.2 107.793998) (end 140.718998 104.275) (width 0.3) (layer F.Cu) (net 19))
 (segment (start 137.2 108.925) (end 137.2 107.793998) (width 0.3) (layer F.Cu) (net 19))
 (segment (start 137.625 62.725) (end 137.85 62.95) (width 0.3) (layer F.Cu) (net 2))
 (segment (start 135.5 62.725) (end 137.625 62.725) (width 0.3) (layer F.Cu) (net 2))
 (segment (start 143.32501 63.77501) (end 142.175 62.625) (width 0.3) (layer F.Cu) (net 2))
 (segment (start 143.32501 70.07499) (end 143.32501 63.77501) (width 0.3) (layer F.Cu) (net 2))
 (segment (start 143.3 70.1) (end 143.32501 70.07499) (width 0.3) (layer F.Cu) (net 2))
 (segment (start 141.85 62.95) (end 142.175 62.625) (width 0.3) (layer F.Cu) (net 2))
 (segment (start 137.85 62.95) (end 141.85 62.95) (width 0.3) (layer F.Cu) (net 2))
 (segment (start 135.575 92.9) (end 136.575 93.9) (width 0.3) (layer F.Cu) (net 2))
 (segment (start 135.575 88.7) (end 135.575 92.9) (width 0.3) (layer F.Cu) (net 2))
 (segment (start 137.515 88.7) (end 137.8 88.415) (width 0.3) (layer F.Cu) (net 2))
 (segment (start 135.575 88.7) (end 137.515 88.7) (width 0.3) (layer F.Cu) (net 2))
 (segment (start 142.025 90.525) (end 143.275 91.775) (width 0.3) (layer F.Cu) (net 2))
 (segment (start 142.025 88.075) (end 142.025 90.525) (width 0.3) (layer F.Cu) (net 2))
 (segment (start 137.815 65.525) (end 137.85 65.49) (width 0.3) (layer F.Cu) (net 3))
 (segment (start 135.5 65.525) (end 137.815 65.525) (width 0.3) (layer F.Cu) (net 3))
 (segment (start 140.5 67.65) (end 142.175 65.975) (width 0.3) (layer F.Cu) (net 3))
 (segment (start 140.5 70.1) (end 140.5 67.65) (width 0.3) (layer F.Cu) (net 3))
 (segment (start 140.01 67.65) (end 140.5 67.65) (width 0.3) (layer F.Cu) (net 3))
 (segment (start 137.85 65.49) (end 140.01 67.65) (width 0.3) (layer F.Cu) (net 3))
 (segment (start 135.6 85.875) (end 135.575 85.9) (width 0.3) (layer F.Cu) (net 1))
 (segment (start 137.8 85.875) (end 135.6 85.875) (width 0.3) (layer F.Cu) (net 1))
 (segment (start 140.875 85.875) (end 142.025 84.725) (width 0.3) (layer F.Cu) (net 1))
 (segment (start 137.8 85.875) (end 140.875 85.875) (width 0.3) (layer F.Cu) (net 1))
 (segment (start 138.99 152.75) (end 136.85 150.61) (width 0.3) (layer F.Cu) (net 6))
 (segment (start 140.825 152.75) (end 138.99 152.75) (width 0.3) (layer F.Cu) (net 6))
 (segment (start 135.22499 106.17501) (end 137.125 104.275) (width 0.3) (layer F.Cu) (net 7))
 (segment (start 135.22499 145.06499) (end 135.22499 106.17501) (width 0.3) (layer F.Cu) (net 7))
 (segment (start 136.85 146.69) (end 135.22499 145.06499) (width 0.3) (layer F.Cu) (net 7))
 (segment (start 137.125 101.775) (end 137.125 104.275) (width 0.3) (layer F.Cu) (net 7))
 (segment (start 138.115 144.614722) (end 138.115 142.68) (width 0.3) (layer F.Cu) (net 10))
 (segment (start 140.314279 146.814001) (end 138.115 144.614722) (width 0.3) (layer F.Cu) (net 10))
 (segment (start 140.963723 146.814001) (end 140.314279 146.814001) (width 0.3) (layer F.Cu) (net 10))
 (segment (start 141.889001 147.739279) (end 140.963723 146.814001) (width 0.3) (layer F.Cu) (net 10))
 (segment (start 141.889001 154.390765) (end 141.889001 147.739279) (width 0.3) (layer F.Cu) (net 10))
 (segment (start 140.459766 155.82) (end 141.889001 154.390765) (width 0.3) (layer F.Cu) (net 10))
 (segment (start 138.115 155.82) (end 140.459766 155.82) (width 0.3) (layer F.Cu) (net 10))
 (segment (start 137.95 96.775) (end 136.575 95.4) (width 0.3) (layer F.Cu) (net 20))
 (segment (start 139.625 96.775) (end 137.95 96.775) (width 0.3) (layer F.Cu) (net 20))
 (segment (start 139.625 137.7) (end 139.625 140.425) (width 0.3) (layer F.Cu) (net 5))
 (segment (start 140.825 141.625) (end 140.825 145.75) (width 0.3) (layer F.Cu) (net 5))
 (segment (start 139.625 140.425) (end 140.825 141.625) (width 0.3) (layer F.Cu) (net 5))
 (segment (start 142.975 122.9625) (end 142.3125 123.625) (width 0.3) (layer F.Cu) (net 5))
 (segment (start 142.975 117.4) (end 142.975 122.9625) (width 0.3) (layer F.Cu) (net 5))
 (segment (start 142.3125 135.0125) (end 142.3125 123.625) (width 0.3) (layer F.Cu) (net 5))
 (segment (start 139.625 137.7) (end 142.3125 135.0125) (width 0.3) (layer F.Cu) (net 5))
 (segment (start 142.975 114.25) (end 142.85 114.125) (width 0.3) (layer F.Cu) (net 5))
 (segment (start 142.975 117.4) (end 142.975 114.25) (width 0.3) (layer F.Cu) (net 5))
 (segment (start 136.25 113.225) (end 136.925 113.9) (width 0.3) (layer F.Cu) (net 5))
 (segment (start 136.25 111.025) (end 136.25 113.225) (width 0.3) (layer F.Cu) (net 5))
 (segment (start 136.925 110.669998) (end 136.925 113.9) (width 0.3) (layer F.Cu) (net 5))
 (segment (start 137.569999 110.024999) (end 136.925 110.669998) (width 0.3) (layer F.Cu) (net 5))
 (segment (start 138.749999 110.024999) (end 137.569999 110.024999) (width 0.3) (layer F.Cu) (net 5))
 (segment (start 142.85 114.125) (end 138.749999 110.024999) (width 0.3) (layer F.Cu) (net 5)))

